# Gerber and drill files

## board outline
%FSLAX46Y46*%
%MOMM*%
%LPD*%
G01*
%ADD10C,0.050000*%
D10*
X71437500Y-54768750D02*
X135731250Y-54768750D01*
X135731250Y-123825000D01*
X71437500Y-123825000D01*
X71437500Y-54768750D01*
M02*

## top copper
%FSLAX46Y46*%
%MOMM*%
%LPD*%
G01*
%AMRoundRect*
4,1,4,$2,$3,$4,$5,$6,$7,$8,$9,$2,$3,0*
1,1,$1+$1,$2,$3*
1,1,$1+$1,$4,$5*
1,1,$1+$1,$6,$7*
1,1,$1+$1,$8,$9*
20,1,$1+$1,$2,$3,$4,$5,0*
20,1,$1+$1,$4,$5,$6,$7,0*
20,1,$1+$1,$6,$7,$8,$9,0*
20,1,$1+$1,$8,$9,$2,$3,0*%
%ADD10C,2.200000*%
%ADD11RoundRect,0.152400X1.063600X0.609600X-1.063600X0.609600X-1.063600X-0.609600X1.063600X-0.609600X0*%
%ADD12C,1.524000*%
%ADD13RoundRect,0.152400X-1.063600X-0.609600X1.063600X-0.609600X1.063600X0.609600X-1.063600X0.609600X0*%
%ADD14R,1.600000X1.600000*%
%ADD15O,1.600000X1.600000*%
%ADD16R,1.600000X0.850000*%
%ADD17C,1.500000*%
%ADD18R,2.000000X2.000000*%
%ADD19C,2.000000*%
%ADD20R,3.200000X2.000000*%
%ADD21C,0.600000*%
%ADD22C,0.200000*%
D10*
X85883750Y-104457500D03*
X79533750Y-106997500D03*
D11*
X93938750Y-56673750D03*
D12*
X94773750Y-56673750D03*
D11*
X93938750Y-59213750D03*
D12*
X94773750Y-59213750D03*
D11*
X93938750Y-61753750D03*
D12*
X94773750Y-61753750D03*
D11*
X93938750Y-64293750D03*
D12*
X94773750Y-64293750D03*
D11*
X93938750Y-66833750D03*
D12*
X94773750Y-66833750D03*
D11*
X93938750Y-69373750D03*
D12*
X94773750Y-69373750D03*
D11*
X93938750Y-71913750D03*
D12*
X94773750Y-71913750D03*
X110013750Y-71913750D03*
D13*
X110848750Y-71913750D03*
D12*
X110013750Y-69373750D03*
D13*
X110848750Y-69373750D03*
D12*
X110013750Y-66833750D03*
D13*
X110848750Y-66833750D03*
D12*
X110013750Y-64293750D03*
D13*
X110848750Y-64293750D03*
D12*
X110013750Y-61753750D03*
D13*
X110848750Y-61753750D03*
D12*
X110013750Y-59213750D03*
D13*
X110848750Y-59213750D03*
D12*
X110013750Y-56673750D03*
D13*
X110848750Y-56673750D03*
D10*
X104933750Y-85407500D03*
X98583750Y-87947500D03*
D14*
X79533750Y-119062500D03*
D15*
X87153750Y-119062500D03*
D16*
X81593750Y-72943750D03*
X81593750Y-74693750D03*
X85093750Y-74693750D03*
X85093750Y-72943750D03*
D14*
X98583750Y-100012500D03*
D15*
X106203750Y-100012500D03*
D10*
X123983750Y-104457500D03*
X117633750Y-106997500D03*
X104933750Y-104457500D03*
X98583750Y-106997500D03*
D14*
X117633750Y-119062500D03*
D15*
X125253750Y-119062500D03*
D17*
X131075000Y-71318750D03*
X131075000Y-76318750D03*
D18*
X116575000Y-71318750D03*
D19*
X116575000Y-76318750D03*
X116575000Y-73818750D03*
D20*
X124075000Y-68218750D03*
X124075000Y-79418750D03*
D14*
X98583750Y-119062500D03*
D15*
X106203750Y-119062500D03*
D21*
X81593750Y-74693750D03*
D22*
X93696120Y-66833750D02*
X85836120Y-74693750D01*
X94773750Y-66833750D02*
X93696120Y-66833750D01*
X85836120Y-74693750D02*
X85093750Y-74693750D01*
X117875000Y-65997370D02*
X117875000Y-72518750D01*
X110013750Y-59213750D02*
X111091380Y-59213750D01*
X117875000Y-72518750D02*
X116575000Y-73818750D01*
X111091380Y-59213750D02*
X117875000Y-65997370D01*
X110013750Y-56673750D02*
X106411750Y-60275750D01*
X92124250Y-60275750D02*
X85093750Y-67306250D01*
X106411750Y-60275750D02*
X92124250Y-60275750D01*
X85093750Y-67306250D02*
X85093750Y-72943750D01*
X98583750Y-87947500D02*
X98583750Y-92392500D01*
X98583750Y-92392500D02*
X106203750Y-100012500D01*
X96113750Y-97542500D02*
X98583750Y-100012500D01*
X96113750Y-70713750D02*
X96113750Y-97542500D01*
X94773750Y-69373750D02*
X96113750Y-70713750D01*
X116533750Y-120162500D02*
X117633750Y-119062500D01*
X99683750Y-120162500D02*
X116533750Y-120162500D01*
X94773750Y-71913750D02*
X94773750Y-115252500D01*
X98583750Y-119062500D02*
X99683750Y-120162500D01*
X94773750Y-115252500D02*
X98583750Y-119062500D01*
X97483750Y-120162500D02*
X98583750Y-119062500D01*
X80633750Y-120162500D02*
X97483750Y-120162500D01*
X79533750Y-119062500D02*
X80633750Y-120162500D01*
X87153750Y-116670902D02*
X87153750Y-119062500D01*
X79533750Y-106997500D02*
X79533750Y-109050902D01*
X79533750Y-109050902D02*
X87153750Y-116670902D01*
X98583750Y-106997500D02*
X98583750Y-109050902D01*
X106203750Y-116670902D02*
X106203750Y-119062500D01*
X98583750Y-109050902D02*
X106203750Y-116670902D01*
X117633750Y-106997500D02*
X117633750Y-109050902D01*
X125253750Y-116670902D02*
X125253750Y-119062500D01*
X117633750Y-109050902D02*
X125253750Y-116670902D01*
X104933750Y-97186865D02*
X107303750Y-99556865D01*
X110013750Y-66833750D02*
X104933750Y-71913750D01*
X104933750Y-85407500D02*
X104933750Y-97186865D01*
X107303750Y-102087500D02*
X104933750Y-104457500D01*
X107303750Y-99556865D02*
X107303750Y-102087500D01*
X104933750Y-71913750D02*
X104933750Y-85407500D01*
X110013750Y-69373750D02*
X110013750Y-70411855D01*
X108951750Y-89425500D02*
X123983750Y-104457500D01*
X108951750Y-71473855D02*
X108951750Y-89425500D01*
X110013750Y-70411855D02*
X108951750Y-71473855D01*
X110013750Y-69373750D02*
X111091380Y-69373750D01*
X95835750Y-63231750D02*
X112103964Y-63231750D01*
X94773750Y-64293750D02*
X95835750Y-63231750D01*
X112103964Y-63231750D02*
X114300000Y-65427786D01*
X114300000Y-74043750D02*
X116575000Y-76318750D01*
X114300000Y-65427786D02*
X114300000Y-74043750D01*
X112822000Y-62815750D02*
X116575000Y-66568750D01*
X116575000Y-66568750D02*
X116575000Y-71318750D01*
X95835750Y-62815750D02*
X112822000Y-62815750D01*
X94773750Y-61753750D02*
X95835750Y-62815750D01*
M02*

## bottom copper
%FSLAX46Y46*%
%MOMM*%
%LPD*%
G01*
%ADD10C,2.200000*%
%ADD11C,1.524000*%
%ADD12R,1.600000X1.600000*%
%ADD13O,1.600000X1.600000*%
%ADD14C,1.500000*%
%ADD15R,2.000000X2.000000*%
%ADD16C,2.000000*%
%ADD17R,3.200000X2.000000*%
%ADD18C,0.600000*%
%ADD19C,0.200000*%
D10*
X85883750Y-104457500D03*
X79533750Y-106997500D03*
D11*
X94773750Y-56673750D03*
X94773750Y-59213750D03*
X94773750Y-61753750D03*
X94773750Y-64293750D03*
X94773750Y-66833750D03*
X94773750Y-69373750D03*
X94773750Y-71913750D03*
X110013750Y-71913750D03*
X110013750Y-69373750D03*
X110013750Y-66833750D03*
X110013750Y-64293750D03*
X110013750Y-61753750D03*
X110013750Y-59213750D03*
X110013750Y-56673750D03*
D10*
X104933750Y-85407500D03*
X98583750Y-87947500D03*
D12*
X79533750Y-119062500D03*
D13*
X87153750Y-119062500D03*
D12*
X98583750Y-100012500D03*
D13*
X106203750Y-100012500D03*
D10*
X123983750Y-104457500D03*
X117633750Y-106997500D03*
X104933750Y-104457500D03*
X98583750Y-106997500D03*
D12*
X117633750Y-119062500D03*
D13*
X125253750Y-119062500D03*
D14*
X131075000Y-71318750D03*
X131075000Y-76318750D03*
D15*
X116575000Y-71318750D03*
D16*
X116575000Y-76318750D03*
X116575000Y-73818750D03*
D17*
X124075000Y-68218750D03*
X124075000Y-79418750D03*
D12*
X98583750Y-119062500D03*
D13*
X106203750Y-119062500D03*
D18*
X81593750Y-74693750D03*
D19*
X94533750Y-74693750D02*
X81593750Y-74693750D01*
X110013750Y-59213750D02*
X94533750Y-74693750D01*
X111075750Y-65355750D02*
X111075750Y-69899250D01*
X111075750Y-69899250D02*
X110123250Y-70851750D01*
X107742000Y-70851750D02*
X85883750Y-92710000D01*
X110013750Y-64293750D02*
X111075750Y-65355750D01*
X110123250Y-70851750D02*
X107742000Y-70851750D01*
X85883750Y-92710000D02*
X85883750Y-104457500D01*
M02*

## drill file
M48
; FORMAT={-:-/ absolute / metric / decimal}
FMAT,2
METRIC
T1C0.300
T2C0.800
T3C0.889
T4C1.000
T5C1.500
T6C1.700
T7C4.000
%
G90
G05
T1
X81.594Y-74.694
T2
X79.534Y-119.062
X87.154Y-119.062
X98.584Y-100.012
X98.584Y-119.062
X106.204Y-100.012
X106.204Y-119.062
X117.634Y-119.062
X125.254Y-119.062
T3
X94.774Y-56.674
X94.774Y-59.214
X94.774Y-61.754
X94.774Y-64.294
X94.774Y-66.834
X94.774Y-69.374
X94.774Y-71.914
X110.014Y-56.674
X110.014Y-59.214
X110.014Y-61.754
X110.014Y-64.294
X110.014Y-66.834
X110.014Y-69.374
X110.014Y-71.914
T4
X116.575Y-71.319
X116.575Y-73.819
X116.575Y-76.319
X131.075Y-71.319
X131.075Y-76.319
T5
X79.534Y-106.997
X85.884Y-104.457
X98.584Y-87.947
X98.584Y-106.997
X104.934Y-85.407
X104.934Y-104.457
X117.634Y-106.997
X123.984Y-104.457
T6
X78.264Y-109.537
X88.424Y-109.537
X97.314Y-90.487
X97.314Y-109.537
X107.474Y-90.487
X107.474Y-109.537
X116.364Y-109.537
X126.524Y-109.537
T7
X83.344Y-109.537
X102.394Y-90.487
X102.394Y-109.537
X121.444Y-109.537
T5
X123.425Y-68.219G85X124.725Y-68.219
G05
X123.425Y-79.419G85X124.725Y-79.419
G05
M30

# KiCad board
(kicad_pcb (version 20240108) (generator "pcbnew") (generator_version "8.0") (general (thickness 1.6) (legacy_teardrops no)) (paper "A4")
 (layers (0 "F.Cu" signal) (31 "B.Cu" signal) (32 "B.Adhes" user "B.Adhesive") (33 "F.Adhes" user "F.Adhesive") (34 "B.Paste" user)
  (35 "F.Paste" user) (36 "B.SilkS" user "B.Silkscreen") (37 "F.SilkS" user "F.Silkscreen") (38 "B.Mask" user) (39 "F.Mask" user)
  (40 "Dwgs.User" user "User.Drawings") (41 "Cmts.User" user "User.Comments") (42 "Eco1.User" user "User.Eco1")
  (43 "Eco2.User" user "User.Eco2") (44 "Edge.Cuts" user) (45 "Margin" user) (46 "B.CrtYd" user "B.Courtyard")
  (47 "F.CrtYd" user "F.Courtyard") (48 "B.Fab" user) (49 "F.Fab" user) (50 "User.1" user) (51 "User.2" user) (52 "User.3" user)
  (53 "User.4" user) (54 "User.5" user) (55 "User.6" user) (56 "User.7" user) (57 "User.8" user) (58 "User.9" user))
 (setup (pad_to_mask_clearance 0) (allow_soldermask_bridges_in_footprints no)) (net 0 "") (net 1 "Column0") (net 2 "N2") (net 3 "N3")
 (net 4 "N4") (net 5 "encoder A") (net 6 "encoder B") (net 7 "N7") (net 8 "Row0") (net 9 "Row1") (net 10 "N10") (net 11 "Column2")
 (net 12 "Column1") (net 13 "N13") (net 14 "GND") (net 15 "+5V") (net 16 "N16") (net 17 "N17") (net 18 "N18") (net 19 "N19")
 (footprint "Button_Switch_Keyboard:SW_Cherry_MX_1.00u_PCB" (layer "F.Cu") (at 85.88375 104.4575)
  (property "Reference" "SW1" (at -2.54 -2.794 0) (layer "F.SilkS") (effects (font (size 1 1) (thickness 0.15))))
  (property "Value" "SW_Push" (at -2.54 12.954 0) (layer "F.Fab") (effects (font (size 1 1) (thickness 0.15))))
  (pad "" np_thru_hole circle (at -7.62 5.08) (size 1.7 1.7) (drill 1.7) (layers "*.Cu" "*.Mask"))
  (pad "" np_thru_hole circle (at -2.54 5.08) (size 4 4) (drill 4) (layers "*.Cu" "*.Mask"))
  (pad "" np_thru_hole circle (at 2.54 5.08) (size 1.7 1.7) (drill 1.7) (layers "*.Cu" "*.Mask"))
  (pad "1" thru_hole circle (at 0 0) (size 2.2 2.2) (drill 1.5) (layers "*.Cu" "*.Mask") (remove_unused_layers no) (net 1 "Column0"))
  (pad "2" thru_hole circle (at -6.35 2.54) (size 2.2 2.2) (drill 1.5) (layers "*.Cu" "*.Mask") (remove_unused_layers no) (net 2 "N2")))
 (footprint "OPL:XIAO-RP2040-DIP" (layer "F.Cu") (at 102.39375 64.29375)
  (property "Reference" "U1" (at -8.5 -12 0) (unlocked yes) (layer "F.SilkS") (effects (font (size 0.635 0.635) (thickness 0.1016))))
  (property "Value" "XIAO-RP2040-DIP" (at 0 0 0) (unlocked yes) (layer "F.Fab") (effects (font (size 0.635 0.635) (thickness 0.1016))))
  (pad "1" smd roundrect (at -8.455 -7.62 180) (size 2.432 1.524) (layers "F.Cu" "F.Mask") (roundrect_rratio 0.1) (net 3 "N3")
   (thermal_bridge_angle 45))
  (pad "1" thru_hole circle (at -7.62 -7.62 180) (size 1.524 1.524) (drill 0.889) (layers "*.Cu" "*.Mask") (remove_unused_layers no)
   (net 3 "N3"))
  (pad "2" smd roundrect (at -8.455 -5.08 180) (size 2.432 1.524) (layers "F.Cu" "F.Mask") (roundrect_rratio 0.1) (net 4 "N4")
   (thermal_bridge_angle 45))
  (pad "2" thru_hole circle (at -7.62 -5.08 180) (size 1.524 1.524) (drill 0.889) (layers "*.Cu" "*.Mask") (remove_unused_layers no)
   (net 4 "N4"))
  (pad "3" smd roundrect (at -8.455 -2.54 180) (size 2.432 1.524) (layers "F.Cu" "F.Mask") (roundrect_rratio 0.1) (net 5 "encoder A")
   (thermal_bridge_angle 45))
  (pad "3" thru_hole circle (at -7.62 -2.54 180) (size 1.524 1.524) (drill 0.889) (layers "*.Cu" "*.Mask") (remove_unused_layers no)
   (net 5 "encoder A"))
  (pad "4" smd roundrect (at -8.455 0 180) (size 2.432 1.524) (layers "F.Cu" "F.Mask") (roundrect_rratio 0.1) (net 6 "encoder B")
   (thermal_bridge_angle 45))
  (pad "4" thru_hole circle (at -7.62 0 180) (size 1.524 1.524) (drill 0.889) (layers "*.Cu" "*.Mask") (remove_unused_layers no)
   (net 6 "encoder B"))
  (pad "5" smd roundrect (at -8.455 2.54 180) (size 2.432 1.524) (layers "F.Cu" "F.Mask") (roundrect_rratio 0.1) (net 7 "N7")
   (thermal_bridge_angle 45))
  (pad "5" thru_hole circle (at -7.62 2.54 180) (size 1.524 1.524) (drill 0.889) (layers "*.Cu" "*.Mask") (remove_unused_layers no)
   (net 7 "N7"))
  (pad "6" smd roundrect (at -8.455 5.08 180) (size 2.432 1.524) (layers "F.Cu" "F.Mask") (roundrect_rratio 0.1) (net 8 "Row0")
   (thermal_bridge_angle 45))
  (pad "6" thru_hole circle (at -7.62 5.08 180) (size 1.524 1.524) (drill 0.889) (layers "*.Cu" "*.Mask") (remove_unused_layers no)
   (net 8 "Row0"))
  (pad "7" smd roundrect (at -8.455 7.62 180) (size 2.432 1.524) (layers "F.Cu" "F.Mask") (roundrect_rratio 0.1) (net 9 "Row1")
   (thermal_bridge_angle 45))
  (pad "7" thru_hole circle (at -7.62 7.62 180) (size 1.524 1.524) (drill 0.889) (layers "*.Cu" "*.Mask") (remove_unused_layers no)
   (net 9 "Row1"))
  (pad "8" thru_hole circle (at 7.62 7.62) (size 1.524 1.524) (drill 0.889) (layers "*.Cu" "*.Mask") (remove_unused_layers no)
   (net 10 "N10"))
  (pad "8" smd roundrect (at 8.455 7.62) (size 2.432 1.524) (layers "F.Cu" "F.Mask") (roundrect_rratio 0.1) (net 10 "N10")
   (thermal_bridge_angle 45))
  (pad "9" thru_hole circle (at 7.62 5.08) (size 1.524 1.524) (drill 0.889) (layers "*.Cu" "*.Mask") (remove_unused_layers no)
   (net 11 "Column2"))
  (pad "9" smd roundrect (at 8.455 5.08) (size 2.432 1.524) (layers "F.Cu" "F.Mask") (roundrect_rratio 0.1) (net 11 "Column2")
   (thermal_bridge_angle 45))
  (pad "10" thru_hole circle (at 7.62 2.54) (size 1.524 1.524) (drill 0.889) (layers "*.Cu" "*.Mask") (remove_unused_layers no)
   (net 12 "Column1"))
  (pad "10" smd roundrect (at 8.455 2.54) (size 2.432 1.524) (layers "F.Cu" "F.Mask") (roundrect_rratio 0.1) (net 12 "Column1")
   (thermal_bridge_angle 45))
  (pad "11" thru_hole circle (at 7.62 0) (size 1.524 1.524) (drill 0.889) (layers "*.Cu" "*.Mask") (remove_unused_layers no)
   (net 1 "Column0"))
  (pad "11" smd roundrect (at 8.455 0) (size 2.432 1.524) (layers "F.Cu" "F.Mask") (roundrect_rratio 0.1) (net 1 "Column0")
   (thermal_bridge_angle 45))
  (pad "12" thru_hole circle (at 7.62 -2.54) (size 1.524 1.524) (drill 0.889) (layers "*.Cu" "*.Mask") (remove_unused_layers no)
   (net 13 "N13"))
  (pad "12" smd roundrect (at 8.455 -2.54) (size 2.432 1.524) (layers "F.Cu" "F.Mask") (roundrect_rratio 0.1) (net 13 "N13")
   (thermal_bridge_angle 45))
  (pad "13" thru_hole circle (at 7.62 -5.08) (size 1.524 1.524) (drill 0.889) (layers "*.Cu" "*.Mask") (remove_unused_layers no)
   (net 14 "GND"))
  (pad "13" smd roundrect (at 8.455 -5.08) (size 2.432 1.524) (layers "F.Cu" "F.Mask") (roundrect_rratio 0.1) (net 14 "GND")
   (thermal_bridge_angle 45))
  (pad "14" thru_hole circle (at 7.62 -7.62) (size 1.524 1.524) (drill 0.889) (layers "*.Cu" "*.Mask") (remove_unused_layers no)
   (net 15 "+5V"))
  (pad "14" smd roundrect (at 8.455 -7.62) (size 2.432 1.524) (layers "F.Cu" "F.Mask") (roundrect_rratio 0.1) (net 15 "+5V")
   (thermal_bridge_angle 45)))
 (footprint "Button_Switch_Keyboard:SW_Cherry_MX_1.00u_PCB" (layer "F.Cu") (at 104.93375 85.4075)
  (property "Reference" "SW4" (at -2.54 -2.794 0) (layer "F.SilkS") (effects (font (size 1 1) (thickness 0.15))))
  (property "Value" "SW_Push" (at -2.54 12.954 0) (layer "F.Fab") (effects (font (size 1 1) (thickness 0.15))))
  (pad "" np_thru_hole circle (at -7.62 5.08) (size 1.7 1.7) (drill 1.7) (layers "*.Cu" "*.Mask"))
  (pad "" np_thru_hole circle (at -2.54 5.08) (size 4 4) (drill 4) (layers "*.Cu" "*.Mask"))
  (pad "" np_thru_hole circle (at 2.54 5.08) (size 1.7 1.7) (drill 1.7) (layers "*.Cu" "*.Mask"))
  (pad "1" thru_hole circle (at 0 0) (size 2.2 2.2) (drill 1.5) (layers "*.Cu" "*.Mask") (remove_unused_layers no) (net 12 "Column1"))
  (pad "2" thru_hole circle (at -6.35 2.54) (size 2.2 2.2) (drill 1.5) (layers "*.Cu" "*.Mask") (remove_unused_layers no) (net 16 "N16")))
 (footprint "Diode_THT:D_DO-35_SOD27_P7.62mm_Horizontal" (layer "F.Cu") (at 79.53375 119.0625)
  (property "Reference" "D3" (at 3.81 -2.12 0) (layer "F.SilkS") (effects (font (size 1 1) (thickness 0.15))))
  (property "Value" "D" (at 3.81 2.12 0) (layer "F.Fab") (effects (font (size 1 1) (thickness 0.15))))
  (pad "1" thru_hole rect (at 0 0) (size 1.6 1.6) (drill 0.8) (layers "*.Cu" "*.Mask") (remove_unused_layers no) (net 9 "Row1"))
  (pad "2" thru_hole oval (at 7.62 0) (size 1.6 1.6) (drill 0.8) (layers "*.Cu" "*.Mask") (remove_unused_layers no) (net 2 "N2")))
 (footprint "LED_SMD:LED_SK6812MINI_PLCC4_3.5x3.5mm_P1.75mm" (layer "F.Cu") (at 83.34375 73.81875)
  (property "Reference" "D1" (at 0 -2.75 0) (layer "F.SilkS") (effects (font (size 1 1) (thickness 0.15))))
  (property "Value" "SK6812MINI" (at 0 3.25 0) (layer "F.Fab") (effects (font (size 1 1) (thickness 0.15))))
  (pad "1" smd rect (at -1.75 -0.875) (size 1.6 0.85) (layers "F.Cu" "F.Paste" "F.Mask") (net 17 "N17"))
  (pad "2" smd rect (at -1.75 0.875) (size 1.6 0.85) (layers "F.Cu" "F.Paste" "F.Mask") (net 14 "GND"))
  (pad "3" smd rect (at 1.75 0.875) (size 1.6 0.85) (layers "F.Cu" "F.Paste" "F.Mask") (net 7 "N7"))
  (pad "4" smd rect (at 1.75 -0.875) (size 1.6 0.85) (layers "F.Cu" "F.Paste" "F.Mask") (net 15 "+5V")))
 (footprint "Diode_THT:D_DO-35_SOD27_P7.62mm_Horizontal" (layer "F.Cu") (at 98.58375 100.0125)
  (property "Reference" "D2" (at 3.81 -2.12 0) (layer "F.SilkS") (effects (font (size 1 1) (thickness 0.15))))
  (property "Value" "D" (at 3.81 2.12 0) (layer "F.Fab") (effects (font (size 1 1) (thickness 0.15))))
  (pad "1" thru_hole rect (at 0 0) (size 1.6 1.6) (drill 0.8) (layers "*.Cu" "*.Mask") (remove_unused_layers no) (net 8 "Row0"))
  (pad "2" thru_hole oval (at 7.62 0) (size 1.6 1.6) (drill 0.8) (layers "*.Cu" "*.Mask") (remove_unused_layers no) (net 16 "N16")))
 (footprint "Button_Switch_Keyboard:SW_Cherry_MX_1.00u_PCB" (layer "F.Cu") (at 123.98375 104.4575)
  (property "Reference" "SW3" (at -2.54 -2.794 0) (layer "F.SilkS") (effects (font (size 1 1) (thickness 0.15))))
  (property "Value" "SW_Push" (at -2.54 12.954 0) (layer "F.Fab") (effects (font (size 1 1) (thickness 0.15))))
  (pad "" np_thru_hole circle (at -7.62 5.08) (size 1.7 1.7) (drill 1.7) (layers "*.Cu" "*.Mask"))
  (pad "" np_thru_hole circle (at -2.54 5.08) (size 4 4) (drill 4) (layers "*.Cu" "*.Mask"))
  (pad "" np_thru_hole circle (at 2.54 5.08) (size 1.7 1.7) (drill 1.7) (layers "*.Cu" "*.Mask"))
  (pad "1" thru_hole circle (at 0 0) (size 2.2 2.2) (drill 1.5) (layers "*.Cu" "*.Mask") (remove_unused_layers no) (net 11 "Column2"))
  (pad "2" thru_hole circle (at -6.35 2.54) (size 2.2 2.2) (drill 1.5) (layers "*.Cu" "*.Mask") (remove_unused_layers no) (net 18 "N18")))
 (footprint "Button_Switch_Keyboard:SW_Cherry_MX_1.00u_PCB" (layer "F.Cu") (at 104.93375 104.4575)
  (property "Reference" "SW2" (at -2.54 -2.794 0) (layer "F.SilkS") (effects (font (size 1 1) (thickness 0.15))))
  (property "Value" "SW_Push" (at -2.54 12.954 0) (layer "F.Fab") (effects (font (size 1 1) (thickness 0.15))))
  (pad "" np_thru_hole circle (at -7.62 5.08) (size 1.7 1.7) (drill 1.7) (layers "*.Cu" "*.Mask"))
  (pad "" np_thru_hole circle (at -2.54 5.08) (size 4 4) (drill 4) (layers "*.Cu" "*.Mask"))
  (pad "" np_thru_hole circle (at 2.54 5.08) (size 1.7 1.7) (drill 1.7) (layers "*.Cu" "*.Mask"))
  (pad "1" thru_hole circle (at 0 0) (size 2.2 2.2) (drill 1.5) (layers "*.Cu" "*.Mask") (remove_unused_layers no) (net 12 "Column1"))
  (pad "2" thru_hole circle (at -6.35 2.54) (size 2.2 2.2) (drill 1.5) (layers "*.Cu" "*.Mask") (remove_unused_layers no) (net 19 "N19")))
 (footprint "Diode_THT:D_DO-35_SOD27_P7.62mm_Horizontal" (layer "F.Cu") (at 117.63375 119.0625)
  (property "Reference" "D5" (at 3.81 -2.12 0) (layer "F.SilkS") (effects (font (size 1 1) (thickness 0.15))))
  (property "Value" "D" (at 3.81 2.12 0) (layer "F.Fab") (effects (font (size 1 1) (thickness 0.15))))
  (pad "1" thru_hole rect (at 0 0) (size 1.6 1.6) (drill 0.8) (layers "*.Cu" "*.Mask") (remove_unused_layers no) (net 9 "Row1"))
  (pad "2" thru_hole oval (at 7.62 0) (size 1.6 1.6) (drill 0.8) (layers "*.Cu" "*.Mask") (remove_unused_layers no) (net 18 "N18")))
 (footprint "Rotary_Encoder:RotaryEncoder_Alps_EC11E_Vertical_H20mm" (layer "F.Cu") (at 116.575 71.31875)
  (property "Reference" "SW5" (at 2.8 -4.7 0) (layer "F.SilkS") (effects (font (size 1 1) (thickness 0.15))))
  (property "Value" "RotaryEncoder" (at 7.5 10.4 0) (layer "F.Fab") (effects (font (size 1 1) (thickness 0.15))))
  (pad "" thru_hole circle (at 14.5 0) (size 1.5 1.5) (drill 1) (layers "*.Cu" "*.Mask") (remove_unused_layers no))
  (pad "" thru_hole circle (at 14.5 5) (size 1.5 1.5) (drill 1) (layers "*.Cu" "*.Mask") (remove_unused_layers no))
  (pad "A" thru_hole rect (at 0 0) (size 2 2) (drill 1) (layers "*.Cu" "*.Mask") (remove_unused_layers no) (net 5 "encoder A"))
  (pad "B" thru_hole circle (at 0 5) (size 2 2) (drill 1) (layers "*.Cu" "*.Mask") (remove_unused_layers no) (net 6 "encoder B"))
  (pad "C" thru_hole circle (at 0 2.5) (size 2 2) (drill 1) (layers "*.Cu" "*.Mask") (remove_unused_layers no) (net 14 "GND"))
  (pad "MP" thru_hole rect (at 7.5 -3.1) (size 3.2 2) (drill oval 2.8 1.5) (layers "*.Cu" "*.Mask") (remove_unused_layers no))
  (pad "MP" thru_hole rect (at 7.5 8.1) (size 3.2 2) (drill oval 2.8 1.5) (layers "*.Cu" "*.Mask") (remove_unused_layers no)))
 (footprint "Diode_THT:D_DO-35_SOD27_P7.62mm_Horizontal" (layer "F.Cu") (at 98.58375 119.0625)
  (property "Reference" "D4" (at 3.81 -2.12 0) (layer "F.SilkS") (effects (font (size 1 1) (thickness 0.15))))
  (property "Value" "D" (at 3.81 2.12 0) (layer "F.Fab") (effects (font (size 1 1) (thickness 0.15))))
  (pad "1" thru_hole rect (at 0 0) (size 1.6 1.6) (drill 0.8) (layers "*.Cu" "*.Mask") (remove_unused_layers no) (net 9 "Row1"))
  (pad "2" thru_hole oval (at 7.62 0) (size 1.6 1.6) (drill 0.8) (layers "*.Cu" "*.Mask") (remove_unused_layers no) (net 19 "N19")))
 (gr_rect (start 71.4375 54.76875) (end 135.73125 123.825) (stroke (width 0.05) (type default)) (fill none) (layer "Edge.Cuts"))
 (segment (start 93.69612 66.83375) (end 85.83612 74.69375) (width 0.2) (layer "F.Cu") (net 7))
 (segment (start 94.77375 66.83375) (end 93.69612 66.83375) (width 0.2) (layer "F.Cu") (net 7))
 (segment (start 85.83612 74.69375) (end 85.09375 74.69375) (width 0.2) (layer "F.Cu") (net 7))
 (segment (start 117.875 65.99737) (end 117.875 72.51875) (width 0.2) (layer "F.Cu") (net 14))
 (segment (start 110.01375 59.21375) (end 111.09138 59.21375) (width 0.2) (layer "F.Cu") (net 14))
 (segment (start 117.875 72.51875) (end 116.575 73.81875) (width 0.2) (layer "F.Cu") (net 14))
 (segment (start 111.09138 59.21375) (end 117.875 65.99737) (width 0.2) (layer "F.Cu") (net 14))
 (via (at 81.59375 74.69375) (size 0.6) (drill 0.3) (layers "F.Cu" "B.Cu") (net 14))
 (segment (start 94.53375 74.69375) (end 81.59375 74.69375) (width 0.2) (layer "B.Cu") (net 14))
 (segment (start 110.01375 59.21375) (end 94.53375 74.69375) (width 0.2) (layer "B.Cu") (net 14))
 (segment (start 110.01375 56.67375) (end 106.41175 60.27575) (width 0.2) (layer "F.Cu") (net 15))
 (segment (start 92.12425 60.27575) (end 85.09375 67.30625) (width 0.2) (layer "F.Cu") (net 15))
 (segment (start 106.41175 60.27575) (end 92.12425 60.27575) (width 0.2) (layer "F.Cu") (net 15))
 (segment (start 85.09375 67.30625) (end 85.09375 72.94375) (width 0.2) (layer "F.Cu") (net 15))
 (segment (start 98.58375 87.9475) (end 98.58375 92.3925) (width 0.2) (layer "F.Cu") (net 16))
 (segment (start 98.58375 92.3925) (end 106.20375 100.0125) (width 0.2) (layer "F.Cu") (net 16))
 (segment (start 96.11375 97.5425) (end 98.58375 100.0125) (width 0.2) (layer "F.Cu") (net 8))
 (segment (start 96.11375 70.71375) (end 96.11375 97.5425) (width 0.2) (layer "F.Cu") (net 8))
 (segment (start 94.77375 69.37375) (end 96.11375 70.71375) (width 0.2) (layer "F.Cu") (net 8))
 (segment (start 116.53375 120.1625) (end 117.63375 119.0625) (width 0.2) (layer "F.Cu") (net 9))
 (segment (start 99.68375 120.1625) (end 116.53375 120.1625) (width 0.2) (layer "F.Cu") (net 9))
 (segment (start 94.77375 71.91375) (end 94.77375 115.2525) (width 0.2) (layer "F.Cu") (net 9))
 (segment (start 98.58375 119.0625) (end 99.68375 120.1625) (width 0.2) (layer "F.Cu") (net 9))
 (segment (start 94.77375 115.2525) (end 98.58375 119.0625) (width 0.2) (layer "F.Cu") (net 9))
 (segment (start 97.48375 120.1625) (end 98.58375 119.0625) (width 0.2) (layer "F.Cu") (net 9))
 (segment (start 80.63375 120.1625) (end 97.48375 120.1625) (width 0.2) (layer "F.Cu") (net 9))
 (segment (start 79.53375 119.0625) (end 80.63375 120.1625) (width 0.2) (layer "F.Cu") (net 9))
 (segment (start 87.15375 116.670902) (end 87.15375 119.0625) (width 0.2) (layer "F.Cu") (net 2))
 (segment (start 79.53375 106.9975) (end 79.53375 109.050902) (width 0.2) (layer "F.Cu") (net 2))
 (segment (start 79.53375 109.050902) (end 87.15375 116.670902) (width 0.2) (layer "F.Cu") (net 2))
 (segment (start 98.58375 106.9975) (end 98.58375 109.050902) (width 0.2) (layer "F.Cu") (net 19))
 (segment (start 106.20375 116.670902) (end 106.20375 119.0625) (width 0.2) (layer "F.Cu") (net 19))
 (segment (start 98.58375 109.050902) (end 106.20375 116.670902) (width 0.2) (layer "F.Cu") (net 19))
 (segment (start 117.63375 106.9975) (end 117.63375 109.050902) (width 0.2) (layer "F.Cu") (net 18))
 (segment (start 125.25375 116.670902) (end 125.25375 119.0625) (width 0.2) (layer "F.Cu") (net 18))
 (segment (start 117.63375 109.050902) (end 125.25375 116.670902) (width 0.2) (layer "F.Cu") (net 18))
 (segment (start 111.07575 65.35575) (end 111.07575 69.89925) (width 0.2) (layer "B.Cu") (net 1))
 (segment (start 111.07575 69.89925) (end 110.12325 70.85175) (width 0.2) (layer "B.Cu") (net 1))
 (segment (start 107.742 70.85175) (end 85.88375 92.71) (width 0.2) (layer "B.Cu") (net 1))
 (segment (start 110.01375 64.29375) (end 111.07575 65.35575) (width 0.2) (layer "B.Cu") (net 1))
 (segment (start 110.12325 70.85175) (end 107.742 70.85175) (width 0.2) (layer "B.Cu") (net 1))
 (segment (start 85.88375 92.71) (end 85.88375 104.4575) (width 0.2) (layer "B.Cu") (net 1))
 (segment (start 104.93375 97.186865) (end 107.30375 99.556865) (width 0.2) (layer "F.Cu") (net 12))
 (segment (start 110.01375 66.83375) (end 104.93375 71.91375) (width 0.2) (layer "F.Cu") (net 12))
 (segment (start 104.93375 85.4075) (end 104.93375 97.186865) (width 0.2) (layer "F.Cu") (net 12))
 (segment (start 107.30375 102.0875) (end 104.93375 104.4575) (width 0.2) (layer "F.Cu") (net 12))
 (segment (start 107.30375 99.556865) (end 107.30375 102.0875) (width 0.2) (layer "F.Cu") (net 12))
 (segment (start 104.93375 71.91375) (end 104.93375 85.4075) (width 0.2) (layer "F.Cu") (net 12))
 (segment (start 110.01375 69.37375) (end 110.01375 70.411855) (width 0.2) (layer "F.Cu") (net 11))
 (segment (start 108.95175 89.4255) (end 123.98375 104.4575) (width 0.2) (layer "F.Cu") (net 11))
 (segment (start 108.95175 71.473855) (end 108.95175 89.4255) (width 0.2) (layer "F.Cu") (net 11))
 (segment (start 110.01375 70.411855) (end 108.95175 71.473855) (width 0.2) (layer "F.Cu") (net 11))
 (segment (start 110.01375 69.37375) (end 111.09138 69.37375) (width 0.2) (layer "F.Cu") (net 11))
 (segment (start 95.83575 63.23175) (end 112.103964 63.23175) (width 0.2) (layer "F.Cu") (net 6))
 (segment (start 94.77375 64.29375) (end 95.83575 63.23175) (width 0.2) (layer "F.Cu") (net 6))
 (segment (start 112.103964 63.23175) (end 114.3 65.427786) (width 0.2) (layer "F.Cu") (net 6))
 (segment (start 114.3 74.04375) (end 116.575 76.31875) (width 0.2) (layer "F.Cu") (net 6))
 (segment (start 114.3 65.427786) (end 114.3 74.04375) (width 0.2) (layer "F.Cu") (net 6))
 (segment (start 112.822 62.81575) (end 116.575 66.56875) (width 0.2) (layer "F.Cu") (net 5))
 (segment (start 116.575 66.56875) (end 116.575 71.31875) (width 0.2) (layer "F.Cu") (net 5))
 (segment (start 95.83575 62.81575) (end 112.822 62.81575) (width 0.2) (layer "F.Cu") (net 5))
 (segment (start 94.77375 61.75375) (end 95.83575 62.81575) (width 0.2) (layer "F.Cu") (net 5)))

